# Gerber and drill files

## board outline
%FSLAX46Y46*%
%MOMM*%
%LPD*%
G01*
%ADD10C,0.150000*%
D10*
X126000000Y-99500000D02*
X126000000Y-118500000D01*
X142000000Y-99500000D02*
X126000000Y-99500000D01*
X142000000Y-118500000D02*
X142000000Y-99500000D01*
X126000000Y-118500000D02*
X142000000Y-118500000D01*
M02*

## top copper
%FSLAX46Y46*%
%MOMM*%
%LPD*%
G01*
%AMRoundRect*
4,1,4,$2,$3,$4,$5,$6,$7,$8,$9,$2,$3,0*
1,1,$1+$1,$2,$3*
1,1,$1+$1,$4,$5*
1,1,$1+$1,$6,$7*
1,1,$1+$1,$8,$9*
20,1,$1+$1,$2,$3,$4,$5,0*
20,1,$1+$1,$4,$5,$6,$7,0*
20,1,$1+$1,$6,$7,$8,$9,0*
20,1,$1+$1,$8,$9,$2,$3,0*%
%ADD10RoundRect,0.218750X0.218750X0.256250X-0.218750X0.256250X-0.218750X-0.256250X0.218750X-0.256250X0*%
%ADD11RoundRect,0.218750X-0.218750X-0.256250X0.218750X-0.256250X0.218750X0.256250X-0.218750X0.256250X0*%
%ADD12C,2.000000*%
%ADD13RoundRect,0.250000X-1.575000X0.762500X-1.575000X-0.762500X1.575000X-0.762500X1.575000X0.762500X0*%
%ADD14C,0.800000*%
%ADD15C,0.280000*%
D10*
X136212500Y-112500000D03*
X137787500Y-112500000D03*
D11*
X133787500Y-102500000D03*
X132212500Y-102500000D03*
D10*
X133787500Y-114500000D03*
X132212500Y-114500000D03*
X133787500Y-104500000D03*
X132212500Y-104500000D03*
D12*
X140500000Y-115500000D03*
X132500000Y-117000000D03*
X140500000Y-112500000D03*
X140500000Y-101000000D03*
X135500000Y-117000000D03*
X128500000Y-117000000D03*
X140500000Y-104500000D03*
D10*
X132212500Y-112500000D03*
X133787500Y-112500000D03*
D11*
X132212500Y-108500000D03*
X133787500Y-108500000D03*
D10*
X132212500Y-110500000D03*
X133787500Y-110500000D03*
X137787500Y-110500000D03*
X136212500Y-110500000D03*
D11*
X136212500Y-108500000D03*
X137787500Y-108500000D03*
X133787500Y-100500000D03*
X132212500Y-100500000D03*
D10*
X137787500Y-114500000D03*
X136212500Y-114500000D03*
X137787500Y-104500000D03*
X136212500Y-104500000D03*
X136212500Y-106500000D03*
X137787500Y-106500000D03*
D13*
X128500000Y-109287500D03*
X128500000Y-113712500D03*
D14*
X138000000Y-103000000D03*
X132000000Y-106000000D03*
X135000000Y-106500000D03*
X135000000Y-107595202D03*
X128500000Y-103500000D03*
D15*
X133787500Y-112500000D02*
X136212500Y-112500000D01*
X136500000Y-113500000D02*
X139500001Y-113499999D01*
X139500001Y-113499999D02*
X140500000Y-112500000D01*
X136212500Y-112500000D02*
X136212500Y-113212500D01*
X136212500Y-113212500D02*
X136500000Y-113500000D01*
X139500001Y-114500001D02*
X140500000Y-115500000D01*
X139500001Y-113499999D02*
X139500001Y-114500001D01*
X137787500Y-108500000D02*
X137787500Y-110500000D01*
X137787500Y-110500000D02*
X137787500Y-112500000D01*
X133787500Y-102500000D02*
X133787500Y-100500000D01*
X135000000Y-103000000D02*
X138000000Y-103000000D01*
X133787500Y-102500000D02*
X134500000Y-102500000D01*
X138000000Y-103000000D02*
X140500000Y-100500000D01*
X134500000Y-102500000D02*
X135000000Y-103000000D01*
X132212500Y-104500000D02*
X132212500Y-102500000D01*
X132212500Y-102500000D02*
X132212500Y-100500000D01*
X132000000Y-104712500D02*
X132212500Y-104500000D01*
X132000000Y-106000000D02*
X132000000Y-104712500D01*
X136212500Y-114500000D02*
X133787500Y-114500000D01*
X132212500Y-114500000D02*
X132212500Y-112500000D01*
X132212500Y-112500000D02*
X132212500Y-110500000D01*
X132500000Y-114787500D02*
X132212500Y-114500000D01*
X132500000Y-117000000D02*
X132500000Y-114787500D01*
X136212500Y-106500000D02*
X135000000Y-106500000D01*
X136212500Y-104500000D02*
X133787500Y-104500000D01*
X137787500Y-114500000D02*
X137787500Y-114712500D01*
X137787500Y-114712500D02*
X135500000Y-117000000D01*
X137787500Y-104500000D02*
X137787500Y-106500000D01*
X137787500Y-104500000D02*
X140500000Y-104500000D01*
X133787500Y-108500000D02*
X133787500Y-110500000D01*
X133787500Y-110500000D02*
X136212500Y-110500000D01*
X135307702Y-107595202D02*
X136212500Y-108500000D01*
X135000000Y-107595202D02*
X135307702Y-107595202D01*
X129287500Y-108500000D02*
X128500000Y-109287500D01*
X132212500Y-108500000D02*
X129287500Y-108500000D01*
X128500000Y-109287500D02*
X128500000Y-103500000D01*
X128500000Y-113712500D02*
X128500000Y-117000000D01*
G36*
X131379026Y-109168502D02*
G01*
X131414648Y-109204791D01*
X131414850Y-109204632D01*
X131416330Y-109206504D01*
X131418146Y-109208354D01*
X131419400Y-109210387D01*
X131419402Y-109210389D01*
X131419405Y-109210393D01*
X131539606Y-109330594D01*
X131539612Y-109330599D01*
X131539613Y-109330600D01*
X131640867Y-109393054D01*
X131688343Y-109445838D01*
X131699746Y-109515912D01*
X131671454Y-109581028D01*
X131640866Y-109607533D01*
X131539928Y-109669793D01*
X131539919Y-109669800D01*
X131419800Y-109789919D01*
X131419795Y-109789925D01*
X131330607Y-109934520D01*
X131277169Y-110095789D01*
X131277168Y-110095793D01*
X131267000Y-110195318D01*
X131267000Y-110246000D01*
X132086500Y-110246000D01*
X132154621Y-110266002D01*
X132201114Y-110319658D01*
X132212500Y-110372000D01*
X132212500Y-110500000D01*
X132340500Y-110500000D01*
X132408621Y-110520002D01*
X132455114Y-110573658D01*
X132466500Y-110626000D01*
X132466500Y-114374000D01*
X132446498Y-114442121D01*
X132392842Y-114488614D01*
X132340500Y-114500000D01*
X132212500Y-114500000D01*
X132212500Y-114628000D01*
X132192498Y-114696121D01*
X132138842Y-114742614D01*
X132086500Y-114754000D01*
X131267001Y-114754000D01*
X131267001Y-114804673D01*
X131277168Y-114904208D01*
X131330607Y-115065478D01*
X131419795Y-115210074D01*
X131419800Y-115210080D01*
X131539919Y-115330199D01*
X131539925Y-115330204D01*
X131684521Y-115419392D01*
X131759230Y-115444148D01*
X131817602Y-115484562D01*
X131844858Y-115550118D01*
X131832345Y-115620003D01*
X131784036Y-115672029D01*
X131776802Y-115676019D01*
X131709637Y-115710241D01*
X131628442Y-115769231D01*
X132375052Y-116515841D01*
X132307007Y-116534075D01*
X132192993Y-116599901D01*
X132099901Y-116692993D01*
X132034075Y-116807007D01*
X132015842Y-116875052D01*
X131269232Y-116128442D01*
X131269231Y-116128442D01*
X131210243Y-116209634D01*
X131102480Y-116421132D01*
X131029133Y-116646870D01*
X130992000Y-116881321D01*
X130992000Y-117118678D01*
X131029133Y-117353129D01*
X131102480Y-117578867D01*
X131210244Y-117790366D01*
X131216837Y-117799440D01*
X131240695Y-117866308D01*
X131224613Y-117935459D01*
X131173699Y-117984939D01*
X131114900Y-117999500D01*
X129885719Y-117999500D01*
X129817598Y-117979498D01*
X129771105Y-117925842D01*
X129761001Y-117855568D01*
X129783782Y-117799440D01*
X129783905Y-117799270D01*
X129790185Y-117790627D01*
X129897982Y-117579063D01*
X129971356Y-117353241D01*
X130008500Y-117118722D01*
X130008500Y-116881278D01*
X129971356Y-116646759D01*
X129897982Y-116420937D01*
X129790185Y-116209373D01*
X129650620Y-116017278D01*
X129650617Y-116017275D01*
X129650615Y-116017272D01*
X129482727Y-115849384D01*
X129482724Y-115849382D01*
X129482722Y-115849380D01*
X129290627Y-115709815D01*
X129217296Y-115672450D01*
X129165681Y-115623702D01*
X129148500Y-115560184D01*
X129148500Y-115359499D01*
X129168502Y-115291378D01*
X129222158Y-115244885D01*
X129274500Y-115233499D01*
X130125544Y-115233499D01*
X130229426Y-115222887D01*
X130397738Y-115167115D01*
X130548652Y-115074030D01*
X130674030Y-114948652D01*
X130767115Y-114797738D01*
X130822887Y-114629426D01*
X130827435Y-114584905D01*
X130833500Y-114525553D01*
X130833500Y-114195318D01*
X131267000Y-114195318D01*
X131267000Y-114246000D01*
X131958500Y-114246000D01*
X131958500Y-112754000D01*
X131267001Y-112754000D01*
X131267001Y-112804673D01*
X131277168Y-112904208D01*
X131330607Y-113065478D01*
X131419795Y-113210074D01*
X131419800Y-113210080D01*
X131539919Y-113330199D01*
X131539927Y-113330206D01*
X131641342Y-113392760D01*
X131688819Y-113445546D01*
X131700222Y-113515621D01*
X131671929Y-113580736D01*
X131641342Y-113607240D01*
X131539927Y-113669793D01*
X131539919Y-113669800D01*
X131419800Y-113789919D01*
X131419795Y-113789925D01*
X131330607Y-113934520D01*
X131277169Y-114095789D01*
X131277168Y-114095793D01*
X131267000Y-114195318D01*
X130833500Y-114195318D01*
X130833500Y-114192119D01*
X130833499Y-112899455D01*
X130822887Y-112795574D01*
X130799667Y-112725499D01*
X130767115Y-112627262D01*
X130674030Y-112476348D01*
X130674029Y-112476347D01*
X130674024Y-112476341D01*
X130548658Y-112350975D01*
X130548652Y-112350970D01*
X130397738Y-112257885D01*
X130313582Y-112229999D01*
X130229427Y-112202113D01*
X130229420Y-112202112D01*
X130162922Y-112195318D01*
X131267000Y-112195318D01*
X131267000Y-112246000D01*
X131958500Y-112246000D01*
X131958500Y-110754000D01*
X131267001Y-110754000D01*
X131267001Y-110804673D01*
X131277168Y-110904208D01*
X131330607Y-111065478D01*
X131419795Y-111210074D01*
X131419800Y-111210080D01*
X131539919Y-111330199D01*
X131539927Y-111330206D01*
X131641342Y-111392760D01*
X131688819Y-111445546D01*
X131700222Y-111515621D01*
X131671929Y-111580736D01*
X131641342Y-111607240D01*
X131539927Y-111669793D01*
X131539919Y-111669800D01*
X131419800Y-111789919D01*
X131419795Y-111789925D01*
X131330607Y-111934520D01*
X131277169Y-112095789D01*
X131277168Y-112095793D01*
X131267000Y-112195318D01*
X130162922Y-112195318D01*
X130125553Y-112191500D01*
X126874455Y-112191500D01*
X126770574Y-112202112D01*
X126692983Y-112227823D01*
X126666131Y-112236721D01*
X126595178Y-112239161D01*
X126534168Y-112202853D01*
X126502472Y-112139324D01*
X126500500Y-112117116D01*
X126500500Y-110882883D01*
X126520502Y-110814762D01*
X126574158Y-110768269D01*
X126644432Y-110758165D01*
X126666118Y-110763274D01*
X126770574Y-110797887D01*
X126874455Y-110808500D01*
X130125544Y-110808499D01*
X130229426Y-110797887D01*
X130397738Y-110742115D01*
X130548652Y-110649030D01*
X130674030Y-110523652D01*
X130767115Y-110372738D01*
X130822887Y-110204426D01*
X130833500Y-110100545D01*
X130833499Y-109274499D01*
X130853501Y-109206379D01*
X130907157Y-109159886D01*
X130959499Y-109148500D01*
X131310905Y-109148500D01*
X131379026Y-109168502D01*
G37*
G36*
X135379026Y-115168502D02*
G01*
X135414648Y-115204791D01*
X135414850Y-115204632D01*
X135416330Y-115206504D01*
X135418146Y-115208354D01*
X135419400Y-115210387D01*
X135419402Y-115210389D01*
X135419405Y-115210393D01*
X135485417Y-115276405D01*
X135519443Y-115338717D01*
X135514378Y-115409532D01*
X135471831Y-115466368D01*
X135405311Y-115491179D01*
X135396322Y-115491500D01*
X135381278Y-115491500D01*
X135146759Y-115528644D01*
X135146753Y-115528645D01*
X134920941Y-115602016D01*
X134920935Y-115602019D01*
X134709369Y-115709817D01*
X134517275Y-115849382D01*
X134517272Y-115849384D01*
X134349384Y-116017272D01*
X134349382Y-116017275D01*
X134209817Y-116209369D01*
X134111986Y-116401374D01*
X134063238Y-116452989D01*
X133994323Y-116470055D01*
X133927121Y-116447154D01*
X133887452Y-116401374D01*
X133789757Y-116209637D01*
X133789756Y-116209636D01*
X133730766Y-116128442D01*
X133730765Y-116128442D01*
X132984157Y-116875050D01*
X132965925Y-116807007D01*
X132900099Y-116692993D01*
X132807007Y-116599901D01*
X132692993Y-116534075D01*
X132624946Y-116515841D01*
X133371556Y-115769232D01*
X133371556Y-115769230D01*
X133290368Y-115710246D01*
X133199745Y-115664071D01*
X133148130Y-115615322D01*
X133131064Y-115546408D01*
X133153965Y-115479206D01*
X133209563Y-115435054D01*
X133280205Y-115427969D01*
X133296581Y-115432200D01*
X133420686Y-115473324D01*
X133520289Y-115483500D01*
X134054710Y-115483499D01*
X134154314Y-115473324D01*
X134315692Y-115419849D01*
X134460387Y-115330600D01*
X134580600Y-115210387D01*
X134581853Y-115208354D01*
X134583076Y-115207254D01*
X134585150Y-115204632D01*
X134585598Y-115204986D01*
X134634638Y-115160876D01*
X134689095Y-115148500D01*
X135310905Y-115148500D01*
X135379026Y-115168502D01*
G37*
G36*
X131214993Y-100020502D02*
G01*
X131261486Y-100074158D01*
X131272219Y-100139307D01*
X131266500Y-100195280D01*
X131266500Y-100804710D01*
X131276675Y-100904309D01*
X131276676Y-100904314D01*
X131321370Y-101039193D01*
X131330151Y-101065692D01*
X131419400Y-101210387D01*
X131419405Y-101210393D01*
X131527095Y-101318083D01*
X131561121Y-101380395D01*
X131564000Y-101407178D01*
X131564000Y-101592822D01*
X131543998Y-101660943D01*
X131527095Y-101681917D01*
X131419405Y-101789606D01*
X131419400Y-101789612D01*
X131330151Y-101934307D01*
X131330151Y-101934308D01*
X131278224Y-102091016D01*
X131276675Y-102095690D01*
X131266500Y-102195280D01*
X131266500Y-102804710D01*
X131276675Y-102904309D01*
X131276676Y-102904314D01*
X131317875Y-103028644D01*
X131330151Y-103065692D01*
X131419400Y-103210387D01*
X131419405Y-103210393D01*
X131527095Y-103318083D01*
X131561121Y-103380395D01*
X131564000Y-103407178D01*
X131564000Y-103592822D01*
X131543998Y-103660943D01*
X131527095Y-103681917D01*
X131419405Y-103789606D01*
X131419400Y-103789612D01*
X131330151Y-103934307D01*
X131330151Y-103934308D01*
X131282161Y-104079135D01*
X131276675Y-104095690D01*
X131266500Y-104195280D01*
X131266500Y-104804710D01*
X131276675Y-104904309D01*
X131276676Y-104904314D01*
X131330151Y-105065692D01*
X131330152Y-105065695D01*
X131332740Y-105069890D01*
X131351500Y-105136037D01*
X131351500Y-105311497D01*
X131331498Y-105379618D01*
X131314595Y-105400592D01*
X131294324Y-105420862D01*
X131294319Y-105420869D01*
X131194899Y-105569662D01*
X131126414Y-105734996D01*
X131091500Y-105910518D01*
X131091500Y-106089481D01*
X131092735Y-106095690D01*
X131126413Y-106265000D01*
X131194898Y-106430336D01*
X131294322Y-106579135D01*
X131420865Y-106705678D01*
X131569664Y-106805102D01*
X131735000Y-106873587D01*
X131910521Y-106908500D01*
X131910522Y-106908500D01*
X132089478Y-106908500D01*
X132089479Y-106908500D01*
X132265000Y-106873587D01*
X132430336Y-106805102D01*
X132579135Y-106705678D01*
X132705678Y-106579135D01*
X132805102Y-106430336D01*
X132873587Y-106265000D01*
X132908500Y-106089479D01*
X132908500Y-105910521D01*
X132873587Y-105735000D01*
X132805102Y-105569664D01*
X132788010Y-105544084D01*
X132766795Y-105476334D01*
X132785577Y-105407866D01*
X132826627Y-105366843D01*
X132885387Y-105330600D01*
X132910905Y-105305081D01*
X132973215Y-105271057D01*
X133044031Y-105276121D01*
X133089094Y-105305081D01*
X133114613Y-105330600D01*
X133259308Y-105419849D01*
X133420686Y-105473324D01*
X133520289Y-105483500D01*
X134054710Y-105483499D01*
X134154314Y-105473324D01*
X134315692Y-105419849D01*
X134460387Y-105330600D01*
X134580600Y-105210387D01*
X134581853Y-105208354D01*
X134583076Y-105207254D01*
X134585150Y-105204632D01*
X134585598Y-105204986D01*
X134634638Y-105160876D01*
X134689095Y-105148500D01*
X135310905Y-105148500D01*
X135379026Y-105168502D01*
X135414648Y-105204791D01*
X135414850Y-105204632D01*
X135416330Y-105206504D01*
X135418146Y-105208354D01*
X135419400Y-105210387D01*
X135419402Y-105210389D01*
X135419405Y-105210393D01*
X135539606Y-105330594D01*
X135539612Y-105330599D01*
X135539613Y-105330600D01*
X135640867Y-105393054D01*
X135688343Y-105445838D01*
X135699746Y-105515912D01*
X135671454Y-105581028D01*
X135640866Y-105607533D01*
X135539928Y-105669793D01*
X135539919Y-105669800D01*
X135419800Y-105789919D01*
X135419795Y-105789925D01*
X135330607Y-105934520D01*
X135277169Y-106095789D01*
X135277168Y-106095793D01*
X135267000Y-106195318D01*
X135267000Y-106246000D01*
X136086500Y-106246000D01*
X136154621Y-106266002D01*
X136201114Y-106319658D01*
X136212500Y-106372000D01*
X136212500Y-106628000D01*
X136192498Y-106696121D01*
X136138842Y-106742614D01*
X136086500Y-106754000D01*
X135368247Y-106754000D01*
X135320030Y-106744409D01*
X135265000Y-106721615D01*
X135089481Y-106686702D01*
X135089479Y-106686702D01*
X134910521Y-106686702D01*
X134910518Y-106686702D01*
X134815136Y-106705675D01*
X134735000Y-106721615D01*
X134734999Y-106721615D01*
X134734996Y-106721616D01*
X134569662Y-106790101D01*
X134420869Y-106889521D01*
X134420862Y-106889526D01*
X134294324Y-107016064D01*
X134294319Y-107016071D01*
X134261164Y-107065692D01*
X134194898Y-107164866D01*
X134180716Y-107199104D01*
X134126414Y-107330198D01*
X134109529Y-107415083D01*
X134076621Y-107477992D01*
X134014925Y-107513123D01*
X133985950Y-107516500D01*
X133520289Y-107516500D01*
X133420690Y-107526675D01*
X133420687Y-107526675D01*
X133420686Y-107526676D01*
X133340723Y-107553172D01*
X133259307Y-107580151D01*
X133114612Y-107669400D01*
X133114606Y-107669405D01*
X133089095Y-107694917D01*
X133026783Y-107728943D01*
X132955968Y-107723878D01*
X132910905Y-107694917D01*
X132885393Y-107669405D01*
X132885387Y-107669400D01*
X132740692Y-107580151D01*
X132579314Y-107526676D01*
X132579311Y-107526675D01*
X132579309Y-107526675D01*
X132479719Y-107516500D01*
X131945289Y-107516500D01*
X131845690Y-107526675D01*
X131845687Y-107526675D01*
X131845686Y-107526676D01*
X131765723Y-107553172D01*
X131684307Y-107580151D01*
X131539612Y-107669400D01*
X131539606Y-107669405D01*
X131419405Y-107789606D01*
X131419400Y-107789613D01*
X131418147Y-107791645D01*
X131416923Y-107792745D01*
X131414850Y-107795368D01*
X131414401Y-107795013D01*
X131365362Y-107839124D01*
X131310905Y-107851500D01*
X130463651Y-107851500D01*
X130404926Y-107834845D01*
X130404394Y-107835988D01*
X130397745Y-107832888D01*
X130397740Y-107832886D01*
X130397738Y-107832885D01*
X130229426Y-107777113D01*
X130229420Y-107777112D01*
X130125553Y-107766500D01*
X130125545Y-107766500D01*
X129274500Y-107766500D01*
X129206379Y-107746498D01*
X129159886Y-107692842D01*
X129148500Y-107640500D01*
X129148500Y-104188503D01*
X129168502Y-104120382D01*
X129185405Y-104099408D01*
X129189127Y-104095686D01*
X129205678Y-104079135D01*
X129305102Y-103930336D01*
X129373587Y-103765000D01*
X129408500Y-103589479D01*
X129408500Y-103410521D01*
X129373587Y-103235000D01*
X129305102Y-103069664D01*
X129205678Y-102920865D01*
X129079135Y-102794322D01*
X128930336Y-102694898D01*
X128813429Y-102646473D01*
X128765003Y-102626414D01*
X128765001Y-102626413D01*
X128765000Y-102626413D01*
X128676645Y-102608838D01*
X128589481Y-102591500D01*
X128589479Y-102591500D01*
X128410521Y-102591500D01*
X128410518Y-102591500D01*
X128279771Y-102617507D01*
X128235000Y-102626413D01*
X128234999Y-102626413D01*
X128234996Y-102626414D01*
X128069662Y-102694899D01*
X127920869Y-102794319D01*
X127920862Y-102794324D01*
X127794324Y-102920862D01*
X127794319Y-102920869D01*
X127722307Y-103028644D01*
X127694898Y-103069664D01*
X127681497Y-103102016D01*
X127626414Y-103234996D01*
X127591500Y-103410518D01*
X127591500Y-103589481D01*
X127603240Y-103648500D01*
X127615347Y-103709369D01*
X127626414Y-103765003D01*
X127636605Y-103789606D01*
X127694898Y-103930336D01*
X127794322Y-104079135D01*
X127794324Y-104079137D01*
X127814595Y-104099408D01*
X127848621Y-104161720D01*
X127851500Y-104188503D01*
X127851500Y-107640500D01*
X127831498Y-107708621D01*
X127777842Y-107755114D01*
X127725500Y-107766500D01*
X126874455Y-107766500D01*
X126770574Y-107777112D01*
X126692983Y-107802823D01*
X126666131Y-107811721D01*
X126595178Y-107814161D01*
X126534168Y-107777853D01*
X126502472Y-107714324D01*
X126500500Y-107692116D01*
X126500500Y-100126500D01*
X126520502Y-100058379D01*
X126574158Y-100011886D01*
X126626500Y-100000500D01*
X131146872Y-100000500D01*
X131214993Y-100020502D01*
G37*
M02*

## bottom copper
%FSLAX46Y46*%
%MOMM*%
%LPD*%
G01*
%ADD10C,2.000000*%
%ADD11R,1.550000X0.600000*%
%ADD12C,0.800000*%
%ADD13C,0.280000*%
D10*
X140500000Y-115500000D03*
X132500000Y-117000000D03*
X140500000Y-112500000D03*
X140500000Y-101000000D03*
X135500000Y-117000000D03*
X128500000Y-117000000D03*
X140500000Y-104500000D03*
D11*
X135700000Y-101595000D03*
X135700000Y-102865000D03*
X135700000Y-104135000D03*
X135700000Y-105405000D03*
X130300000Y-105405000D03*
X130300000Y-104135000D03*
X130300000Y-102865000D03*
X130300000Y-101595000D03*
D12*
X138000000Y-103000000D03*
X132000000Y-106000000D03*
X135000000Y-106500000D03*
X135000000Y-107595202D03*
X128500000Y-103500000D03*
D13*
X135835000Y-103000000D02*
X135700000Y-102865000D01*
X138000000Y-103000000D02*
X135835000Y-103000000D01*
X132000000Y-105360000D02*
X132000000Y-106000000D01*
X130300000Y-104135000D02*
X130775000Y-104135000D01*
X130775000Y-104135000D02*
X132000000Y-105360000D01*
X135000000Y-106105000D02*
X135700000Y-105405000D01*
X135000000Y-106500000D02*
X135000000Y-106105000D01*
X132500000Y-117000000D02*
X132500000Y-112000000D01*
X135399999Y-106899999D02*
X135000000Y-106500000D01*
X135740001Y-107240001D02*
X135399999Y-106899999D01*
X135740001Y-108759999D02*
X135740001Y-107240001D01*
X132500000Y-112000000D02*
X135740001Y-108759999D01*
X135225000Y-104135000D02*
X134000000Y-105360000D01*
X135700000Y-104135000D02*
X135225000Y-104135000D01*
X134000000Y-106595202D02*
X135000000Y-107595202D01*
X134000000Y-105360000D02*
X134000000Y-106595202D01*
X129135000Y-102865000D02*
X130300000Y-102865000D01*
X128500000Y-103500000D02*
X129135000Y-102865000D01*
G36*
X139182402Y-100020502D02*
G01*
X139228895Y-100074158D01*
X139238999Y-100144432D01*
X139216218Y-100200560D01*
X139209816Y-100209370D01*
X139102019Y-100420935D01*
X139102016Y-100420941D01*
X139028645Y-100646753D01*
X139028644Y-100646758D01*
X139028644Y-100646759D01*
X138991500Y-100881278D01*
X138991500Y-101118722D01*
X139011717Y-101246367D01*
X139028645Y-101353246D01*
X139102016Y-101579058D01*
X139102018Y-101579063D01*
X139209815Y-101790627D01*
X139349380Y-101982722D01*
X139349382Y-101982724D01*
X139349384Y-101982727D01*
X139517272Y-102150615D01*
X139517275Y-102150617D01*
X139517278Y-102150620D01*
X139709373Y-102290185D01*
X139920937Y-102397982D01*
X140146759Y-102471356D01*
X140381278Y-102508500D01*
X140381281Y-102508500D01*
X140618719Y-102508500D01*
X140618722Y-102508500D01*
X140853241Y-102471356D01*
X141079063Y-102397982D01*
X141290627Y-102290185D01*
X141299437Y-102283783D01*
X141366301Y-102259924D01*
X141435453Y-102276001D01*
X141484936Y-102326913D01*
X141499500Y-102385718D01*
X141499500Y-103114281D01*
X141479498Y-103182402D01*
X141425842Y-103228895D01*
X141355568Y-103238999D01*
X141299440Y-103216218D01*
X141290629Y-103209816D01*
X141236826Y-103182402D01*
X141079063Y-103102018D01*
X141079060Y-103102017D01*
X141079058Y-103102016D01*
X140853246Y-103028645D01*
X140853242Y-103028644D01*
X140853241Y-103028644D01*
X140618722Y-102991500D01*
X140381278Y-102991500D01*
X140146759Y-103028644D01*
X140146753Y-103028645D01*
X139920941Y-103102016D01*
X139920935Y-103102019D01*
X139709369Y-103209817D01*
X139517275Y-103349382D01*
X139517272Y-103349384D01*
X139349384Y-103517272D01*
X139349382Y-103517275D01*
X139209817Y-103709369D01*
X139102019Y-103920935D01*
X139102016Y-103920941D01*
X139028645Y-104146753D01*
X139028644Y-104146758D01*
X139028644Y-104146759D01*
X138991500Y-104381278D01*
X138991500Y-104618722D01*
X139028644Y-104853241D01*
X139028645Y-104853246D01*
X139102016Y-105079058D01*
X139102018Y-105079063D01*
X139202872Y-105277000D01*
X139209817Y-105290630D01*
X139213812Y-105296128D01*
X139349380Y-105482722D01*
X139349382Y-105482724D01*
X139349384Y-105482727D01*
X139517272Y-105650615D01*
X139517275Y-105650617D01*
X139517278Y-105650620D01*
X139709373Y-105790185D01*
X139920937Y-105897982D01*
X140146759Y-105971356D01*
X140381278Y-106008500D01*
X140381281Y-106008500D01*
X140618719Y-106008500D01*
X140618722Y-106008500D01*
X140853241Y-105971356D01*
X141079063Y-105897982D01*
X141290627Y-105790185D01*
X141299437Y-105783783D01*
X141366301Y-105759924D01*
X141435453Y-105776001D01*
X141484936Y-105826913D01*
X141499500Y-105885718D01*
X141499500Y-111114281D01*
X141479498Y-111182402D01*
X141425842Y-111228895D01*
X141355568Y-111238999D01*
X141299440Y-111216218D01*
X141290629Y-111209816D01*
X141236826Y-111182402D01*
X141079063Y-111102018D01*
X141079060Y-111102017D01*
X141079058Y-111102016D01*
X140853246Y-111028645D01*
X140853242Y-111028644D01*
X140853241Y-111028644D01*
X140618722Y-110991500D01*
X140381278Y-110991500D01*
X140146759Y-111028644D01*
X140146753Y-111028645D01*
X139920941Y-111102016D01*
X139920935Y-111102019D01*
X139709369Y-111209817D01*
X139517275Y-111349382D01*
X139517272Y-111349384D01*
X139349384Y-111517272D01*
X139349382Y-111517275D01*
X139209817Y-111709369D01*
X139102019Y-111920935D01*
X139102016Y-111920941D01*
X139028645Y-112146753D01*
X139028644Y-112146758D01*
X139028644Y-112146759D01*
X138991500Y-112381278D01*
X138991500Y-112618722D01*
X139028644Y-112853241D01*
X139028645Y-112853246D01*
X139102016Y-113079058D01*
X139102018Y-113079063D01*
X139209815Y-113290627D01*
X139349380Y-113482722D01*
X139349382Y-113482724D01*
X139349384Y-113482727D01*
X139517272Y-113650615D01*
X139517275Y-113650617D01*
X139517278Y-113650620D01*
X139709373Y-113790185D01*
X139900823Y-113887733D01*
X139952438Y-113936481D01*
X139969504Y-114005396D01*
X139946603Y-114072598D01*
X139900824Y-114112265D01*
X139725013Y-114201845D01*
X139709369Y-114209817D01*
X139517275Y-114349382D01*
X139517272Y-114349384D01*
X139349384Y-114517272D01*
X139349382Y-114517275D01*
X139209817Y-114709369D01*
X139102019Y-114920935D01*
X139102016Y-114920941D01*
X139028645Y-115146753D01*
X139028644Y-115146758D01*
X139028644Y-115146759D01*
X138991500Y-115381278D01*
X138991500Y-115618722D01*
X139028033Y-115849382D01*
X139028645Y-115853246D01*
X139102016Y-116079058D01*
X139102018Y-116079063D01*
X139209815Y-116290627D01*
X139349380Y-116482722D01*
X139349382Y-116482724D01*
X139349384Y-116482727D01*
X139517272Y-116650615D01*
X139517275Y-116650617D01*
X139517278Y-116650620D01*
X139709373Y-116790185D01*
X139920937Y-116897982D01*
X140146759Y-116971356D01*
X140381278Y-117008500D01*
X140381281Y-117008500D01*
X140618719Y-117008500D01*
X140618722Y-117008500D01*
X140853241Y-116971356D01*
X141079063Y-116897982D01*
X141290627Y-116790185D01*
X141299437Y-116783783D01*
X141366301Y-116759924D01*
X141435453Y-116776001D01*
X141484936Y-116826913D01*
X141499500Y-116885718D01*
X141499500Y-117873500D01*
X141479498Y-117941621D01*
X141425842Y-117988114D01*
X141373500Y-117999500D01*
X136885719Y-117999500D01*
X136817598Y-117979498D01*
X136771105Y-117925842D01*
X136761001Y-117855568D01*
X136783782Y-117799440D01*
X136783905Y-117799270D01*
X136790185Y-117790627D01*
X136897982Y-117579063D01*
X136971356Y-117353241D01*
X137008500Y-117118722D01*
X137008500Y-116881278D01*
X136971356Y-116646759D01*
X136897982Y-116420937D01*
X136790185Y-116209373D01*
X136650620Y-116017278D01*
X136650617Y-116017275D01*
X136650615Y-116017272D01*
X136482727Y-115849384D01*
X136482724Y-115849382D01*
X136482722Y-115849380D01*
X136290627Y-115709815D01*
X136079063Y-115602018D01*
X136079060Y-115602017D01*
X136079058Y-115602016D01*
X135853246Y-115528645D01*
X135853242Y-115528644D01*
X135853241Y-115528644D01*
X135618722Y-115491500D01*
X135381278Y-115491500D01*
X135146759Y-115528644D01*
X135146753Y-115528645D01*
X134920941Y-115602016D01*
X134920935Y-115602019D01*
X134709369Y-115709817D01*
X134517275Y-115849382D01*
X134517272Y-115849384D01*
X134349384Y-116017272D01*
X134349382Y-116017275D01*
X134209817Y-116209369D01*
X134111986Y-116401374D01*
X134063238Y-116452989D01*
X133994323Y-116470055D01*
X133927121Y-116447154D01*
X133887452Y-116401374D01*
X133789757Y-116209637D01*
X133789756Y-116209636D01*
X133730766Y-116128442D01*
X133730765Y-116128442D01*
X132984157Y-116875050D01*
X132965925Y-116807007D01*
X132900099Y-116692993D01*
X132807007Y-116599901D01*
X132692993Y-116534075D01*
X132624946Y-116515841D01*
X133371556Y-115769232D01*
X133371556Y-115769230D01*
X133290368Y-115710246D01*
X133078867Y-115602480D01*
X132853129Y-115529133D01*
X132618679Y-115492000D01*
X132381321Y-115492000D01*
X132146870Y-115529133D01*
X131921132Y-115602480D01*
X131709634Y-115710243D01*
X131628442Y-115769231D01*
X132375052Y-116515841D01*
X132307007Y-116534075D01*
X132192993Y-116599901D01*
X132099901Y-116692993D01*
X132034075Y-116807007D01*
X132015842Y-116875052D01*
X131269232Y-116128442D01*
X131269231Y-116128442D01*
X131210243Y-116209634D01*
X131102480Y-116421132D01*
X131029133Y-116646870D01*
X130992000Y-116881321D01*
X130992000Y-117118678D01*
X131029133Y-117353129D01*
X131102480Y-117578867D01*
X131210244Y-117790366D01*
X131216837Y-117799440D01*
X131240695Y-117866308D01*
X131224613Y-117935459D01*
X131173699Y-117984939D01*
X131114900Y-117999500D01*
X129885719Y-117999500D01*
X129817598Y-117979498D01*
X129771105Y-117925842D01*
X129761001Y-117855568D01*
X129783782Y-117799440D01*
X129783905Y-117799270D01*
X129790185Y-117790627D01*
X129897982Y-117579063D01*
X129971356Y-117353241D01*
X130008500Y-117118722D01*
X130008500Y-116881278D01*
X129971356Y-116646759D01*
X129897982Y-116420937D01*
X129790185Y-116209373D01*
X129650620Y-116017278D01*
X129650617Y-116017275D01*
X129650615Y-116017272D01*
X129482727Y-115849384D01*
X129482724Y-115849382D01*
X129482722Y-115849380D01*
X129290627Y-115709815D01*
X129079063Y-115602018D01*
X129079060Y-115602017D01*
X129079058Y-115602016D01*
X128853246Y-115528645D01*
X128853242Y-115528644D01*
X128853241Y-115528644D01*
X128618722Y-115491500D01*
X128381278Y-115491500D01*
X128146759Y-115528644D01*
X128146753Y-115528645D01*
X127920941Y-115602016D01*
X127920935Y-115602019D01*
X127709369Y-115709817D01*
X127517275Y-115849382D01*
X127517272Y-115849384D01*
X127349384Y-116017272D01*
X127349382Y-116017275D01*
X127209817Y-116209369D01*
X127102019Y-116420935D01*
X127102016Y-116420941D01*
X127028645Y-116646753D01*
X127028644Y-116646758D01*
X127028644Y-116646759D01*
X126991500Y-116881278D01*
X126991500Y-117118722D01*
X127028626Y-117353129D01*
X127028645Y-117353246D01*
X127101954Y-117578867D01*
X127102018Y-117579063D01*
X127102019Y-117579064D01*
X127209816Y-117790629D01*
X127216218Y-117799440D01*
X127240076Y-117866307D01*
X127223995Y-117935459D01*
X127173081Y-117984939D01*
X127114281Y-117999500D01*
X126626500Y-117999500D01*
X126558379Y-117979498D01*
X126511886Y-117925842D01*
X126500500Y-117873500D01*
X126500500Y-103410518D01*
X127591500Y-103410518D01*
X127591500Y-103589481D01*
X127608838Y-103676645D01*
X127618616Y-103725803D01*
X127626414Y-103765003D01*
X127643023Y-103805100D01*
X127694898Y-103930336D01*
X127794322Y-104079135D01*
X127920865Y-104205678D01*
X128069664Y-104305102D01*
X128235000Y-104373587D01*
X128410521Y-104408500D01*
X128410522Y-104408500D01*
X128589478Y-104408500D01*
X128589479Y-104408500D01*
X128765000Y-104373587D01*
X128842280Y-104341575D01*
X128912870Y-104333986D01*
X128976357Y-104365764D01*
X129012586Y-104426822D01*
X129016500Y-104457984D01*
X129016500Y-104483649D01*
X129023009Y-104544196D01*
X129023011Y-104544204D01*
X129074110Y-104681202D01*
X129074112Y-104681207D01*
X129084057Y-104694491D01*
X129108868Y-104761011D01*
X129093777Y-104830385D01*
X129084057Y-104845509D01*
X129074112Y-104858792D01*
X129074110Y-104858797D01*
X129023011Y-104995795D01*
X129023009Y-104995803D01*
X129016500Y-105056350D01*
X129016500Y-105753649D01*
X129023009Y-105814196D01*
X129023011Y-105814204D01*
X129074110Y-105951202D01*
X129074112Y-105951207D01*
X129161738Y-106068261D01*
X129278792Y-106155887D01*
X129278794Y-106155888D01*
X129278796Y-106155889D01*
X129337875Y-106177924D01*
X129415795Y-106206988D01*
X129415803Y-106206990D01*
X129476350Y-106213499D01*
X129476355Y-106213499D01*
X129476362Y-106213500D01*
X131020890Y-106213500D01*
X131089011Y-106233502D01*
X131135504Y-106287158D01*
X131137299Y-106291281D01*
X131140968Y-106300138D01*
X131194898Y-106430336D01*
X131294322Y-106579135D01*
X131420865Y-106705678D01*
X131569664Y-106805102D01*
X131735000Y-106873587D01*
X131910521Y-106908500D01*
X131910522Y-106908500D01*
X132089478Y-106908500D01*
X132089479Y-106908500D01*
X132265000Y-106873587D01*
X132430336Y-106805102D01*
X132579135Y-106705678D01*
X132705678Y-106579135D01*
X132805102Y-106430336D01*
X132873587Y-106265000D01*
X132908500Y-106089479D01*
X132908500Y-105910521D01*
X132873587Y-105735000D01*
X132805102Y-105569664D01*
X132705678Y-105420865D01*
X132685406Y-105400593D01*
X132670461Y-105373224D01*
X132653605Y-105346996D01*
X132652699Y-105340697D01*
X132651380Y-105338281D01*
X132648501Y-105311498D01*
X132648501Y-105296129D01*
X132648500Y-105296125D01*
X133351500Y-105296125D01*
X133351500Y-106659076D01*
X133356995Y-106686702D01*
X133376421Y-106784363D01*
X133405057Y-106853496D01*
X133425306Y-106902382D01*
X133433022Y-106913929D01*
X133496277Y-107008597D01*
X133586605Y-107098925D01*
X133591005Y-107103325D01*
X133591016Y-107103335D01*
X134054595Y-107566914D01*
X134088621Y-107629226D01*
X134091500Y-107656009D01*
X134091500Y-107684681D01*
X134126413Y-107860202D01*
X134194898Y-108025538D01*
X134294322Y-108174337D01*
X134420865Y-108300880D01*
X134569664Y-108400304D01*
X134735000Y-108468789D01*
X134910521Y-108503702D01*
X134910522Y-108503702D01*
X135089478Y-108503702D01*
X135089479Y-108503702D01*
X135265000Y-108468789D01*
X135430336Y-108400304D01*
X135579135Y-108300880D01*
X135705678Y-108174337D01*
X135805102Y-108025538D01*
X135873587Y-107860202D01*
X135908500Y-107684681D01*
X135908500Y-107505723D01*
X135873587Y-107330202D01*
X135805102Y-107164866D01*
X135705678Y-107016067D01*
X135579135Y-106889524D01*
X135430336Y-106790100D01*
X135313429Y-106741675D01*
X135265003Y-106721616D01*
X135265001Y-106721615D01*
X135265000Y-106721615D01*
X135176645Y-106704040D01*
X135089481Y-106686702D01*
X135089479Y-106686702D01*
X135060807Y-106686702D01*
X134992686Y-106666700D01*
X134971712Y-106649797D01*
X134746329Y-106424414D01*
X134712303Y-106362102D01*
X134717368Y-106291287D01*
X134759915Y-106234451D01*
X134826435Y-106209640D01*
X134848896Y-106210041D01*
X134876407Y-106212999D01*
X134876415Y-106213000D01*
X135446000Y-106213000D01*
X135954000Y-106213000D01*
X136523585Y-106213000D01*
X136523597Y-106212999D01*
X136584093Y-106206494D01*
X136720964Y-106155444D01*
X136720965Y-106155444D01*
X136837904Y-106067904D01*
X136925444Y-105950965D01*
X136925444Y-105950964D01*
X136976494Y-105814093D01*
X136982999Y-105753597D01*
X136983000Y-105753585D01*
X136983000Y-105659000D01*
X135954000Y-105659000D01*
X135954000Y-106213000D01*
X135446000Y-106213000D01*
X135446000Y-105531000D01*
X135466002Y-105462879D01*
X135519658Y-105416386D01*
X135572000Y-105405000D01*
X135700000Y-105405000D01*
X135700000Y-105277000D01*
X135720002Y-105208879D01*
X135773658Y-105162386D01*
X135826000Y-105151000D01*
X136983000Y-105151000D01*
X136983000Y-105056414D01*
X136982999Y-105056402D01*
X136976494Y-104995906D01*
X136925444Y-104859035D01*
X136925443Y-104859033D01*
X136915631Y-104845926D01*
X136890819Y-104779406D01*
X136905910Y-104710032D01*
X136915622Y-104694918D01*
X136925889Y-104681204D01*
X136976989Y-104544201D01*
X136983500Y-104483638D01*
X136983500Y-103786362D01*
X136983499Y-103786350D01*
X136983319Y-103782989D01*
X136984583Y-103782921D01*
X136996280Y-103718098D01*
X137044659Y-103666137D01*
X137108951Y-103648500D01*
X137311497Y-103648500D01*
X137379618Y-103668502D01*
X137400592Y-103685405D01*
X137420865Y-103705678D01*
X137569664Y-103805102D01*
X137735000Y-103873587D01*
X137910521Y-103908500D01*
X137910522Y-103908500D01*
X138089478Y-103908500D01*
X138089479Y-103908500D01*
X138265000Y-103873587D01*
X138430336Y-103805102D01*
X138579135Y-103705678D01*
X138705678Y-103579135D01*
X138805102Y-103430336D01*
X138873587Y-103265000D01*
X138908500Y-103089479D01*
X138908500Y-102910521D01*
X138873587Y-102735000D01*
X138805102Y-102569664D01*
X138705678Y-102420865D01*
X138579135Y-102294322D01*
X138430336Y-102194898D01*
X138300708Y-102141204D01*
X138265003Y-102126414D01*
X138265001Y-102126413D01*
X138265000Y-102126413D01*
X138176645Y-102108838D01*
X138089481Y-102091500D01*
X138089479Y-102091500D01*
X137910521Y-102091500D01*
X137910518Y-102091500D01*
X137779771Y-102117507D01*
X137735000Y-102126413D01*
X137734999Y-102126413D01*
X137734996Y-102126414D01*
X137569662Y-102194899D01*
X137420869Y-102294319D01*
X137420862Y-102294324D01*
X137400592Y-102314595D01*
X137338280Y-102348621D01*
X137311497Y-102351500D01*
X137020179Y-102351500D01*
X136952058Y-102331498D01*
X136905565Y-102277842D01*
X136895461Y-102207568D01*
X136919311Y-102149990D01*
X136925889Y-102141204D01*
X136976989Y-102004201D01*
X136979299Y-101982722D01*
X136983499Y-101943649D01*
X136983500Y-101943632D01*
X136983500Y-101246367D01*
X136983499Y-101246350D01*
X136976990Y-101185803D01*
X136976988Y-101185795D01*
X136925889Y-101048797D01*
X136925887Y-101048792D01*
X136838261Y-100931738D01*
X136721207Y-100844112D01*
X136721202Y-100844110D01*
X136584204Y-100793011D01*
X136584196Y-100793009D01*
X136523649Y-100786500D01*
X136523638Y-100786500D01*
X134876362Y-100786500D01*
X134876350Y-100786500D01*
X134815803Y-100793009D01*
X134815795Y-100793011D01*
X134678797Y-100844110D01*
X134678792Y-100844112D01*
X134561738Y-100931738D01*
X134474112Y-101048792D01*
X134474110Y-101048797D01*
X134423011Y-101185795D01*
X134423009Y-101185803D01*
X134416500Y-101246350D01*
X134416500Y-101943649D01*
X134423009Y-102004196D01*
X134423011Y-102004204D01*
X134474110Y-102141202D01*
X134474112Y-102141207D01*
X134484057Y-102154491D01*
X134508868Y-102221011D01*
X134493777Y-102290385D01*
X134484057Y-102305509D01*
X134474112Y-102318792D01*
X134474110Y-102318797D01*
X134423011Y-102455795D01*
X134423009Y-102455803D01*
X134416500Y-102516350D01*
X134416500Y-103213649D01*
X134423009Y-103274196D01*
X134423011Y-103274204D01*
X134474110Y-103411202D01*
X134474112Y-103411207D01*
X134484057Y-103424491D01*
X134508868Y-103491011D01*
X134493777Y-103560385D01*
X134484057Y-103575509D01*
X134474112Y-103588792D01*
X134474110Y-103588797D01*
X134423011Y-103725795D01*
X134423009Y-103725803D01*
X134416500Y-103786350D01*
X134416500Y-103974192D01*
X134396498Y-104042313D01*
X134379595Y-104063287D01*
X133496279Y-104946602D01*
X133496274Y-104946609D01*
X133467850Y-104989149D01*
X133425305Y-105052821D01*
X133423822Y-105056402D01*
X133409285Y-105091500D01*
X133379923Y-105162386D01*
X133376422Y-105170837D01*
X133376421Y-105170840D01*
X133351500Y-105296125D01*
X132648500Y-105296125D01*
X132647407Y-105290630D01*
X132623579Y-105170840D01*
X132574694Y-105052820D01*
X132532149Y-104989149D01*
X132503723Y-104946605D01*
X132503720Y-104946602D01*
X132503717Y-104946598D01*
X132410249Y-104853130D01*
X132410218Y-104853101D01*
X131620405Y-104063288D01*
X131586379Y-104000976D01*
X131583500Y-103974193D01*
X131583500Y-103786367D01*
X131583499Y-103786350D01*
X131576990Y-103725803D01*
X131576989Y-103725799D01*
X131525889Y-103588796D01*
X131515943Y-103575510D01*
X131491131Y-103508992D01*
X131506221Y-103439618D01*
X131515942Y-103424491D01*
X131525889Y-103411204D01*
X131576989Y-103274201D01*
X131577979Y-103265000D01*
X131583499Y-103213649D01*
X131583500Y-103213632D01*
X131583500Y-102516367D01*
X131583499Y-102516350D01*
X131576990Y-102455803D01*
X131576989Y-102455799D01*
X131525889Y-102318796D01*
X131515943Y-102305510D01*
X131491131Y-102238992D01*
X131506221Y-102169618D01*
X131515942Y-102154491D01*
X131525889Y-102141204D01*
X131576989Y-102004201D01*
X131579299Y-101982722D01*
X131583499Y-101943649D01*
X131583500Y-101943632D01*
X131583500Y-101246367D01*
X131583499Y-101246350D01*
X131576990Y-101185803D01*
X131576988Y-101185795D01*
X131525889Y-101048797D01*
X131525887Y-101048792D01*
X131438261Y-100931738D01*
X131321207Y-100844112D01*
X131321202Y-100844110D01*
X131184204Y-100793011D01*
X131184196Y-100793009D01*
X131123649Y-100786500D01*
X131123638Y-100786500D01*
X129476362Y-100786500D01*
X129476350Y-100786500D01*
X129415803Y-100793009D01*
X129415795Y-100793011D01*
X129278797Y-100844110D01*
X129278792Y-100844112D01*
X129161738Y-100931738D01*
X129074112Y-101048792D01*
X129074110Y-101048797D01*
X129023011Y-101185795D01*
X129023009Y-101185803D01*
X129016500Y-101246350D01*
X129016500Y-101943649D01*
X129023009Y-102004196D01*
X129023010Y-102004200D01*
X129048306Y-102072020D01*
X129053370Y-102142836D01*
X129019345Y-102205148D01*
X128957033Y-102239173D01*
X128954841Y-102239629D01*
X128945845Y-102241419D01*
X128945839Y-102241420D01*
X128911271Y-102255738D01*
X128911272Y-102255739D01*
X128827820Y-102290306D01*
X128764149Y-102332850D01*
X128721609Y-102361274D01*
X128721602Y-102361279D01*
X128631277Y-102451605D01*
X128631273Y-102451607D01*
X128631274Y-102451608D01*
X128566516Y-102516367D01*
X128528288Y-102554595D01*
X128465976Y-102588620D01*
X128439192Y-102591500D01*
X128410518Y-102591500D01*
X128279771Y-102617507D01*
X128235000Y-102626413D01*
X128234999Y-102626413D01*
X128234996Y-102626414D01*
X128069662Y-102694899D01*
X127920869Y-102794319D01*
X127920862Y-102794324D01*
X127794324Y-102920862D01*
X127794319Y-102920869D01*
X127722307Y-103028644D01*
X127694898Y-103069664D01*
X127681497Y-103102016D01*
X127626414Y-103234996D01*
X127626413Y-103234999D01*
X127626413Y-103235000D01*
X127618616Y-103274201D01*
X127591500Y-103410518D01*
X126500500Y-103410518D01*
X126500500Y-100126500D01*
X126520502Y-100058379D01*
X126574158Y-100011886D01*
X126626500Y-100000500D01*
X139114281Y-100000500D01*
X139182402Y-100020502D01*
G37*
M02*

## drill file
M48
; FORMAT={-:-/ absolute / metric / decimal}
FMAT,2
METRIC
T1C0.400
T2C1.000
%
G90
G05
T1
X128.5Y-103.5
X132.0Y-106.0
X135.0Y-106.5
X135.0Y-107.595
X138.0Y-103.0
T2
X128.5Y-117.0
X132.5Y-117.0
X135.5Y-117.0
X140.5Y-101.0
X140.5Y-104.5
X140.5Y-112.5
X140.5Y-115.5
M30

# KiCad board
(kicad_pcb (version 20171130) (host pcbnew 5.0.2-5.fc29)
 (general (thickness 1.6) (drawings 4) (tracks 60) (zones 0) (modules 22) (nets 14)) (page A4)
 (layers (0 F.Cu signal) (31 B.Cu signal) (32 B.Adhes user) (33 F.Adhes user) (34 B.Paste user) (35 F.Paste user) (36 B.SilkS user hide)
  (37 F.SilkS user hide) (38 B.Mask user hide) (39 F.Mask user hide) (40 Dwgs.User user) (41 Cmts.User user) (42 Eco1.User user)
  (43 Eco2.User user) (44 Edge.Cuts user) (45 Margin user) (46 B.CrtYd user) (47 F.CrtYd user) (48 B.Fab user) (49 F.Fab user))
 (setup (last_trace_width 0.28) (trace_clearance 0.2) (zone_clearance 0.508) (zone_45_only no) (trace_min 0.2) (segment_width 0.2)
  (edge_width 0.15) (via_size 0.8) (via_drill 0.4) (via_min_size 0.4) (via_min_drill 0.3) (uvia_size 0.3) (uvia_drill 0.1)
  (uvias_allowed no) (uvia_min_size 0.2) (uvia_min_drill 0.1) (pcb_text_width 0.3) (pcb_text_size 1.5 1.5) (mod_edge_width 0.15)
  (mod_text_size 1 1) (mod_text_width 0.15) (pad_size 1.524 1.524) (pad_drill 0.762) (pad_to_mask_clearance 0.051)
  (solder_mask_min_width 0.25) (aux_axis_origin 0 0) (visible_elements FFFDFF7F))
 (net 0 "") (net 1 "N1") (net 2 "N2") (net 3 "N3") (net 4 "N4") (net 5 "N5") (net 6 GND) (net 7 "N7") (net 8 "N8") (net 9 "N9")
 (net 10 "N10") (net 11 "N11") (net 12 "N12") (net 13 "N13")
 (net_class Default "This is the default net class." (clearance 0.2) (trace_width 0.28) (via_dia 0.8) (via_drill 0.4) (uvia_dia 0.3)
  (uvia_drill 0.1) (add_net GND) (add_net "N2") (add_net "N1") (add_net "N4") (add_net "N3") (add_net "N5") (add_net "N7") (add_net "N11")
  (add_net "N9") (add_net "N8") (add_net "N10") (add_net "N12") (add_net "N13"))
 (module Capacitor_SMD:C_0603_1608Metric (layer F.Cu) (at 137 112.5 180)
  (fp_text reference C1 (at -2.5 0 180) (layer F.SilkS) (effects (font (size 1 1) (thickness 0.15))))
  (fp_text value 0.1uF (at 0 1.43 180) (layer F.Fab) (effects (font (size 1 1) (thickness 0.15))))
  (pad 2 smd roundrect (at 0.7875 0 180) (size 0.875 0.95) (layers F.Cu F.Paste F.Mask) (roundrect_rratio 0.25) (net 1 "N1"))
  (pad 1 smd roundrect (at -0.7875 0 180) (size 0.875 0.95) (layers F.Cu F.Paste F.Mask) (roundrect_rratio 0.25) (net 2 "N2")))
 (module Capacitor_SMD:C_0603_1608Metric (layer F.Cu) (at 133 102.5)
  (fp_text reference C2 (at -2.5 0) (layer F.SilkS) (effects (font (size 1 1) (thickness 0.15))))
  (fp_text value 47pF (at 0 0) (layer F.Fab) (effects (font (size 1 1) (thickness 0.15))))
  (pad 2 smd roundrect (at 0.7875 0) (size 0.875 0.95) (layers F.Cu F.Paste F.Mask) (roundrect_rratio 0.25) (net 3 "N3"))
  (pad 1 smd roundrect (at -0.7875 0) (size 0.875 0.95) (layers F.Cu F.Paste F.Mask) (roundrect_rratio 0.25) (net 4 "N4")))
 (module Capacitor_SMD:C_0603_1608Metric (layer F.Cu) (at 133 114.5 180)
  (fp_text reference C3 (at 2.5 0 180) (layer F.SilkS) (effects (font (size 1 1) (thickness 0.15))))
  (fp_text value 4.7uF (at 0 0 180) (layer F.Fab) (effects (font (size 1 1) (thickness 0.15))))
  (pad 1 smd roundrect (at -0.7875 0 180) (size 0.875 0.95) (layers F.Cu F.Paste F.Mask) (roundrect_rratio 0.25) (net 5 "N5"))
  (pad 2 smd roundrect (at 0.7875 0 180) (size 0.875 0.95) (layers F.Cu F.Paste F.Mask) (roundrect_rratio 0.25) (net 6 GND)))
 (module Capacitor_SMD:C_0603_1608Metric (layer F.Cu) (at 133 104.5 180)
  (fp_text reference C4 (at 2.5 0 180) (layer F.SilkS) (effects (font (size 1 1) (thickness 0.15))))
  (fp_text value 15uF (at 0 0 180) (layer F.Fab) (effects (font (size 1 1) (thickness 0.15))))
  (pad 1 smd roundrect (at -0.7875 0 180) (size 0.875 0.95) (layers F.Cu F.Paste F.Mask) (roundrect_rratio 0.25) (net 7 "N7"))
  (pad 2 smd roundrect (at 0.7875 0 180) (size 0.875 0.95) (layers F.Cu F.Paste F.Mask) (roundrect_rratio 0.25) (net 4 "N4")))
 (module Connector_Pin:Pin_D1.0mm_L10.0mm (layer F.Cu) (at 140.5 115.5)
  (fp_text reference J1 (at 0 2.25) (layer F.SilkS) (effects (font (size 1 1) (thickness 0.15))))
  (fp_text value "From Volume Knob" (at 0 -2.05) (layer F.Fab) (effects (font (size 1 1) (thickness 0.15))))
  (pad 1 thru_hole circle (at 0 0) (size 2 2) (drill 1) (layers *.Cu *.Mask) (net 1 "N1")))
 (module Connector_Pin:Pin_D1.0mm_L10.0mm (layer F.Cu) (at 132.5 117)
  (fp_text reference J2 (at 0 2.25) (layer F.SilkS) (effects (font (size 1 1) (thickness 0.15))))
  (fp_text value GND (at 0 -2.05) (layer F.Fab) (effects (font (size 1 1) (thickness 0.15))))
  (pad 1 thru_hole circle (at 0 0) (size 2 2) (drill 1) (layers *.Cu *.Mask) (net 6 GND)))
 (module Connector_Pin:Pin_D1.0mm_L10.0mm (layer F.Cu) (at 140.5 112.5)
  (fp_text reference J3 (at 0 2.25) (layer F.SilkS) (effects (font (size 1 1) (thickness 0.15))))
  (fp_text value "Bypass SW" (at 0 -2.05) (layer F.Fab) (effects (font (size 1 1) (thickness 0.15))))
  (pad 1 thru_hole circle (at 0 0) (size 2 2) (drill 1) (layers *.Cu *.Mask) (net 1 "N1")))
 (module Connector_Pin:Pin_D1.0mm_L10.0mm (layer F.Cu) (at 140.5 101)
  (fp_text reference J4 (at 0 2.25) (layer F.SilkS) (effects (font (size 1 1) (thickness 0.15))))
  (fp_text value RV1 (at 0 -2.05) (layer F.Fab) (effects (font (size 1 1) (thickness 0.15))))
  (pad 1 thru_hole circle (at 0 0) (size 2 2) (drill 1) (layers *.Cu *.Mask) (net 3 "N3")))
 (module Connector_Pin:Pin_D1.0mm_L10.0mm (layer F.Cu) (at 135.5 117)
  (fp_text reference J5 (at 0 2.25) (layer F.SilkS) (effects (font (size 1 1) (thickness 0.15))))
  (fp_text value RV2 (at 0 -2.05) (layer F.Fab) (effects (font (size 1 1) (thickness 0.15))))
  (pad 1 thru_hole circle (at 0 0) (size 2 2) (drill 1) (layers *.Cu *.Mask) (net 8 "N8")))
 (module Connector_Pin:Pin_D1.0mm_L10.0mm (layer F.Cu) (at 128.5 117)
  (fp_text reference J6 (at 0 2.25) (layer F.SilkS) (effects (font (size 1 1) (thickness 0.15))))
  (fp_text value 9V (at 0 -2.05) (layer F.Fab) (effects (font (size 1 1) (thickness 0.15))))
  (pad 1 thru_hole circle (at 0 0) (size 2 2) (drill 1) (layers *.Cu *.Mask) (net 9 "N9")))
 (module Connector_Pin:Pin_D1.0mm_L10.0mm (layer F.Cu) (at 140.5 104.5)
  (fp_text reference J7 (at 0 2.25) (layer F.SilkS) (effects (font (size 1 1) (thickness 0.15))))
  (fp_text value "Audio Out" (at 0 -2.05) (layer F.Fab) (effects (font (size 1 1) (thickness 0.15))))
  (pad 1 thru_hole circle (at 0 0) (size 2 2) (drill 1) (layers *.Cu *.Mask) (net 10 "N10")))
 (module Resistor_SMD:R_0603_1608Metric (layer F.Cu) (at 133 112.5 180)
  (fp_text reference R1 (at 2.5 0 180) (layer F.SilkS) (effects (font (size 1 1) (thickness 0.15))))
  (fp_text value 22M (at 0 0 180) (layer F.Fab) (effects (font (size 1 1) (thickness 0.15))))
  (pad 2 smd roundrect (at 0.7875 0 180) (size 0.875 0.95) (layers F.Cu F.Paste F.Mask) (roundrect_rratio 0.25) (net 6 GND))
  (pad 1 smd roundrect (at -0.7875 0 180) (size 0.875 0.95) (layers F.Cu F.Paste F.Mask) (roundrect_rratio 0.25) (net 1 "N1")))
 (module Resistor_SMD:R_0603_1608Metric (layer F.Cu) (at 133 108.5)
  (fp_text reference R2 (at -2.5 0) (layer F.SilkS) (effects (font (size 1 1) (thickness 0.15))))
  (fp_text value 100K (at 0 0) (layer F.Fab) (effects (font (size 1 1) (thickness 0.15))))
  (pad 1 smd roundrect (at -0.7875 0) (size 0.875 0.95) (layers F.Cu F.Paste F.Mask) (roundrect_rratio 0.25) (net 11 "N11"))
  (pad 2 smd roundrect (at 0.7875 0) (size 0.875 0.95) (layers F.Cu F.Paste F.Mask) (roundrect_rratio 0.25) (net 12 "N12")))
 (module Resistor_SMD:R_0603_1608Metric (layer F.Cu) (at 133 110.5 180)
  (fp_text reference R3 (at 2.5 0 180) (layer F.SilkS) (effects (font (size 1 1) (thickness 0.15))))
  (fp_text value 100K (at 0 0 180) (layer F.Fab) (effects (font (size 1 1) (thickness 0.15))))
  (pad 2 smd roundrect (at 0.7875 0 180) (size 0.875 0.95) (layers F.Cu F.Paste F.Mask) (roundrect_rratio 0.25) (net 6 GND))
  (pad 1 smd roundrect (at -0.7875 0 180) (size 0.875 0.95) (layers F.Cu F.Paste F.Mask) (roundrect_rratio 0.25) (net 12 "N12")))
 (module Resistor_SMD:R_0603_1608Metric (layer F.Cu) (at 137 110.5 180)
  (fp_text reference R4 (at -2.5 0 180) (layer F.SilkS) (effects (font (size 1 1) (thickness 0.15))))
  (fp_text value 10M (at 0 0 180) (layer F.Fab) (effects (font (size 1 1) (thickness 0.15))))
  (pad 1 smd roundrect (at -0.7875 0 180) (size 0.875 0.95) (layers F.Cu F.Paste F.Mask) (roundrect_rratio 0.25) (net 2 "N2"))
  (pad 2 smd roundrect (at 0.7875 0 180) (size 0.875 0.95) (layers F.Cu F.Paste F.Mask) (roundrect_rratio 0.25) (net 12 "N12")))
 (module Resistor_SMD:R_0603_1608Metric (layer F.Cu) (at 137 108.5)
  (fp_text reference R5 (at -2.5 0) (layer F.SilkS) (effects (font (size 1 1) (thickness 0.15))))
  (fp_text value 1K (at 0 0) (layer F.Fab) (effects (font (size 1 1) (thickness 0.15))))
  (pad 1 smd roundrect (at -0.7875 0) (size 0.875 0.95) (layers F.Cu F.Paste F.Mask) (roundrect_rratio 0.25) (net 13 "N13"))
  (pad 2 smd roundrect (at 0.7875 0) (size 0.875 0.95) (layers F.Cu F.Paste F.Mask) (roundrect_rratio 0.25) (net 2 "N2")))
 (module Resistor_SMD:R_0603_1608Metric (layer F.Cu) (at 133 100.5)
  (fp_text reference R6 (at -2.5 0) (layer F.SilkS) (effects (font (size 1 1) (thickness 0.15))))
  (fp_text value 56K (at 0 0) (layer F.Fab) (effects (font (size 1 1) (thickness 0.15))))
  (pad 2 smd roundrect (at 0.7875 0) (size 0.875 0.95) (layers F.Cu F.Paste F.Mask) (roundrect_rratio 0.25) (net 3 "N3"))
  (pad 1 smd roundrect (at -0.7875 0) (size 0.875 0.95) (layers F.Cu F.Paste F.Mask) (roundrect_rratio 0.25) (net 4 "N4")))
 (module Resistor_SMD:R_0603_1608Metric (layer F.Cu) (at 137 114.5 180)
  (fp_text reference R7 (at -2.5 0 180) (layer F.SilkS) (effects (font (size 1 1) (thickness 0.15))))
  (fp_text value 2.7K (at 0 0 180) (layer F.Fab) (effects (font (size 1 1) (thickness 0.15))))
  (pad 1 smd roundrect (at -0.7875 0 180) (size 0.875 0.95) (layers F.Cu F.Paste F.Mask) (roundrect_rratio 0.25) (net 8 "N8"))
  (pad 2 smd roundrect (at 0.7875 0 180) (size 0.875 0.95) (layers F.Cu F.Paste F.Mask) (roundrect_rratio 0.25) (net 5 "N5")))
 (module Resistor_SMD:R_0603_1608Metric (layer F.Cu) (at 137 104.5 180)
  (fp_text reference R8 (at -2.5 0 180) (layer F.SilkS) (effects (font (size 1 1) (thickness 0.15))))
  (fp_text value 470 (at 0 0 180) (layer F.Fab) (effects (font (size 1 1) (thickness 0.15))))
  (pad 1 smd roundrect (at -0.7875 0 180) (size 0.875 0.95) (layers F.Cu F.Paste F.Mask) (roundrect_rratio 0.25) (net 10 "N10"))
  (pad 2 smd roundrect (at 0.7875 0 180) (size 0.875 0.95) (layers F.Cu F.Paste F.Mask) (roundrect_rratio 0.25) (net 7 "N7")))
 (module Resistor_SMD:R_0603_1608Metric (layer F.Cu) (at 137 106.5 180)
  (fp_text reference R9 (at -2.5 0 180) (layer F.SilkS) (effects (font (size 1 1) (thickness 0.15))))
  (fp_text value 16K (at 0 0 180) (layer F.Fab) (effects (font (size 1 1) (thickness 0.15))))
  (pad 2 smd roundrect (at 0.7875 0 180) (size 0.875 0.95) (layers F.Cu F.Paste F.Mask) (roundrect_rratio 0.25) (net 6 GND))
  (pad 1 smd roundrect (at -0.7875 0 180) (size 0.875 0.95) (layers F.Cu F.Paste F.Mask) (roundrect_rratio 0.25) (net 10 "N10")))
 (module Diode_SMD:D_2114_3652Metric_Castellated (layer F.Cu) (at 128.5 111.5 270)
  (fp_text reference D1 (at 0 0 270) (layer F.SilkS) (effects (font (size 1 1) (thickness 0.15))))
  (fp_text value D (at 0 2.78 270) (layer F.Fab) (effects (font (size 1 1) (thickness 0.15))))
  (pad 1 smd roundrect (at -2.2125 0 270) (size 2.025 3.65) (layers F.Cu F.Paste F.Mask) (roundrect_rratio 0.123457) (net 11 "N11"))
  (pad 2 smd roundrect (at 2.2125 0 270) (size 2.025 3.65) (layers F.Cu F.Paste F.Mask) (roundrect_rratio 0.123457) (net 9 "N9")))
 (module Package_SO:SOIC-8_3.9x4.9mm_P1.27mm (layer B.Cu) (at 133 103.5 180)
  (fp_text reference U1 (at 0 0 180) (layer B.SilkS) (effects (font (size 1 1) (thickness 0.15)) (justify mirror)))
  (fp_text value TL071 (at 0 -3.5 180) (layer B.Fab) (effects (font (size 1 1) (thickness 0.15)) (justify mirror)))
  (pad 1 smd rect (at -2.7 1.905 180) (size 1.55 0.6) (layers B.Cu B.Paste B.Mask))
  (pad 2 smd rect (at -2.7 0.635 180) (size 1.55 0.6) (layers B.Cu B.Paste B.Mask) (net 3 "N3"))
  (pad 3 smd rect (at -2.7 -0.635 180) (size 1.55 0.6) (layers B.Cu B.Paste B.Mask) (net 13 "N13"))
  (pad 4 smd rect (at -2.7 -1.905 180) (size 1.55 0.6) (layers B.Cu B.Paste B.Mask) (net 6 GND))
  (pad 5 smd rect (at 2.7 -1.905 180) (size 1.55 0.6) (layers B.Cu B.Paste B.Mask))
  (pad 6 smd rect (at 2.7 -0.635 180) (size 1.55 0.6) (layers B.Cu B.Paste B.Mask) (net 4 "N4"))
  (pad 7 smd rect (at 2.7 0.635 180) (size 1.55 0.6) (layers B.Cu B.Paste B.Mask) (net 11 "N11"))
  (pad 8 smd rect (at 2.7 1.905 180) (size 1.55 0.6) (layers B.Cu B.Paste B.Mask)))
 (gr_line (start 126 99.5) (end 126 118.5) (layer Edge.Cuts) (width 0.15))
 (gr_line (start 142 99.5) (end 126 99.5) (layer Edge.Cuts) (width 0.15))
 (gr_line (start 142 118.5) (end 142 99.5) (layer Edge.Cuts) (width 0.15))
 (gr_line (start 126 118.5) (end 142 118.5) (layer Edge.Cuts) (width 0.15))
 (segment (start 133.7875 112.5) (end 136.2125 112.5) (width 0.28) (layer F.Cu) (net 1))
 (segment (start 136.5 113.5) (end 139.500001 113.499999) (width 0.28) (layer F.Cu) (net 1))
 (segment (start 139.500001 113.499999) (end 140.5 112.5) (width 0.28) (layer F.Cu) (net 1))
 (segment (start 136.2125 112.5) (end 136.2125 113.2125) (width 0.28) (layer F.Cu) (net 1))
 (segment (start 136.2125 113.2125) (end 136.5 113.5) (width 0.28) (layer F.Cu) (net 1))
 (segment (start 139.500001 114.500001) (end 140.5 115.5) (width 0.28) (layer F.Cu) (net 1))
 (segment (start 139.500001 113.499999) (end 139.500001 114.500001) (width 0.28) (layer F.Cu) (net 1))
 (segment (start 137.7875 108.5) (end 137.7875 110.5) (width 0.28) (layer F.Cu) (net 2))
 (segment (start 137.7875 110.5) (end 137.7875 112.5) (width 0.28) (layer F.Cu) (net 2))
 (segment (start 133.7875 102.5) (end 133.7875 100.5) (width 0.28) (layer F.Cu) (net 3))
 (segment (start 135 103) (end 138 103) (width 0.28) (layer F.Cu) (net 3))
 (segment (start 133.7875 102.5) (end 134.5 102.5) (width 0.28) (layer F.Cu) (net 3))
 (segment (start 138 103) (end 140.5 100.5) (width 0.28) (layer F.Cu) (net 3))
 (segment (start 134.5 102.5) (end 135 103) (width 0.28) (layer F.Cu) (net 3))
 (via (at 138 103) (size 0.8) (drill 0.4) (layers F.Cu B.Cu) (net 3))
 (segment (start 135.835 103) (end 135.7 102.865) (width 0.28) (layer B.Cu) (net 3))
 (segment (start 138 103) (end 135.835 103) (width 0.28) (layer B.Cu) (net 3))
 (segment (start 132.2125 104.5) (end 132.2125 102.5) (width 0.28) (layer F.Cu) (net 4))
 (segment (start 132.2125 102.5) (end 132.2125 100.5) (width 0.28) (layer F.Cu) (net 4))
 (segment (start 132 105.36) (end 132 106) (width 0.28) (layer B.Cu) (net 4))
 (via (at 132 106) (size 0.8) (drill 0.4) (layers F.Cu B.Cu) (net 4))
 (segment (start 130.3 104.135) (end 130.775 104.135) (width 0.28) (layer B.Cu) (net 4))
 (segment (start 130.775 104.135) (end 132 105.36) (width 0.28) (layer B.Cu) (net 4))
 (segment (start 132 104.7125) (end 132.2125 104.5) (width 0.28) (layer F.Cu) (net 4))
 (segment (start 132 106) (end 132 104.7125) (width 0.28) (layer F.Cu) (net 4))
 (segment (start 136.2125 114.5) (end 133.7875 114.5) (width 0.28) (layer F.Cu) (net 5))
 (segment (start 132.2125 114.5) (end 132.2125 112.5) (width 0.28) (layer F.Cu) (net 6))
 (segment (start 132.2125 112.5) (end 132.2125 110.5) (width 0.28) (layer F.Cu) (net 6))
 (segment (start 132.5 114.7875) (end 132.2125 114.5) (width 0.28) (layer F.Cu) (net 6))
 (segment (start 132.5 117) (end 132.5 114.7875) (width 0.28) (layer F.Cu) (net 6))
 (segment (start 136.2125 106.5) (end 135 106.5) (width 0.28) (layer F.Cu) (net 6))
 (via (at 135 106.5) (size 0.8) (drill 0.4) (layers F.Cu B.Cu) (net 6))
 (segment (start 135 106.105) (end 135.7 105.405) (width 0.28) (layer B.Cu) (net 6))
 (segment (start 135 106.5) (end 135 106.105) (width 0.28) (layer B.Cu) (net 6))
 (segment (start 132.5 117) (end 132.5 112) (width 0.28) (layer B.Cu) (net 6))
 (segment (start 135.399999 106.899999) (end 135 106.5) (width 0.28) (layer B.Cu) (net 6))
 (segment (start 135.740001 107.240001) (end 135.399999 106.899999) (width 0.28) (layer B.Cu) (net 6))
 (segment (start 135.740001 108.759999) (end 135.740001 107.240001) (width 0.28) (layer B.Cu) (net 6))
 (segment (start 132.5 112) (end 135.740001 108.759999) (width 0.28) (layer B.Cu) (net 6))
 (segment (start 136.2125 104.5) (end 133.7875 104.5) (width 0.28) (layer F.Cu) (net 7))
 (segment (start 137.7875 114.5) (end 137.7875 114.7125) (width 0.28) (layer F.Cu) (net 8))
 (segment (start 137.7875 114.7125) (end 135.5 117) (width 0.28) (layer F.Cu) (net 8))
 (segment (start 137.7875 104.5) (end 137.7875 106.5) (width 0.28) (layer F.Cu) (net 10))
 (segment (start 137.7875 104.5) (end 140.5 104.5) (width 0.28) (layer F.Cu) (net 10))
 (segment (start 133.7875 108.5) (end 133.7875 110.5) (width 0.28) (layer F.Cu) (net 12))
 (segment (start 133.7875 110.5) (end 136.2125 110.5) (width 0.28) (layer F.Cu) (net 12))
 (segment (start 135.225 104.135) (end 134 105.36) (width 0.28) (layer B.Cu) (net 13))
 (segment (start 135.7 104.135) (end 135.225 104.135) (width 0.28) (layer B.Cu) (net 13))
 (segment (start 134 106.595202) (end 135 107.595202) (width 0.28) (layer B.Cu) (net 13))
 (segment (start 134 105.36) (end 134 106.595202) (width 0.28) (layer B.Cu) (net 13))
 (via (at 135 107.595202) (size 0.8) (drill 0.4) (layers F.Cu B.Cu) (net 13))
 (segment (start 135.307702 107.595202) (end 136.2125 108.5) (width 0.28) (layer F.Cu) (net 13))
 (segment (start 135 107.595202) (end 135.307702 107.595202) (width 0.28) (layer F.Cu) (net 13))
 (segment (start 129.2875 108.5) (end 128.5 109.2875) (width 0.28) (layer F.Cu) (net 11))
 (segment (start 132.2125 108.5) (end 129.2875 108.5) (width 0.28) (layer F.Cu) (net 11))
 (segment (start 128.5 109.2875) (end 128.5 103.5) (width 0.28) (layer F.Cu) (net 11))
 (via (at 128.5 103.5) (size 0.8) (drill 0.4) (layers F.Cu B.Cu) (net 11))
 (segment (start 129.135 102.865) (end 130.3 102.865) (width 0.28) (layer B.Cu) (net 11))
 (segment (start 128.5 103.5) (end 129.135 102.865) (width 0.28) (layer B.Cu) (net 11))
 (segment (start 128.5 113.7125) (end 128.5 117) (width 0.28) (layer F.Cu) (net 9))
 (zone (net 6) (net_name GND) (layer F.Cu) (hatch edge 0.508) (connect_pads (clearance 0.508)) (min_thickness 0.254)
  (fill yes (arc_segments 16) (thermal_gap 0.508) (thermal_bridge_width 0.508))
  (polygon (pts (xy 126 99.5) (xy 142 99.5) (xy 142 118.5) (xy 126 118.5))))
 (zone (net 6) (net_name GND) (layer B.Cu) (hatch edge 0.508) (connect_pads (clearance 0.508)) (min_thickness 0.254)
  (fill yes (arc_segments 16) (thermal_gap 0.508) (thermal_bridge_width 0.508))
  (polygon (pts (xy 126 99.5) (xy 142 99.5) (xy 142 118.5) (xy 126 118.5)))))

